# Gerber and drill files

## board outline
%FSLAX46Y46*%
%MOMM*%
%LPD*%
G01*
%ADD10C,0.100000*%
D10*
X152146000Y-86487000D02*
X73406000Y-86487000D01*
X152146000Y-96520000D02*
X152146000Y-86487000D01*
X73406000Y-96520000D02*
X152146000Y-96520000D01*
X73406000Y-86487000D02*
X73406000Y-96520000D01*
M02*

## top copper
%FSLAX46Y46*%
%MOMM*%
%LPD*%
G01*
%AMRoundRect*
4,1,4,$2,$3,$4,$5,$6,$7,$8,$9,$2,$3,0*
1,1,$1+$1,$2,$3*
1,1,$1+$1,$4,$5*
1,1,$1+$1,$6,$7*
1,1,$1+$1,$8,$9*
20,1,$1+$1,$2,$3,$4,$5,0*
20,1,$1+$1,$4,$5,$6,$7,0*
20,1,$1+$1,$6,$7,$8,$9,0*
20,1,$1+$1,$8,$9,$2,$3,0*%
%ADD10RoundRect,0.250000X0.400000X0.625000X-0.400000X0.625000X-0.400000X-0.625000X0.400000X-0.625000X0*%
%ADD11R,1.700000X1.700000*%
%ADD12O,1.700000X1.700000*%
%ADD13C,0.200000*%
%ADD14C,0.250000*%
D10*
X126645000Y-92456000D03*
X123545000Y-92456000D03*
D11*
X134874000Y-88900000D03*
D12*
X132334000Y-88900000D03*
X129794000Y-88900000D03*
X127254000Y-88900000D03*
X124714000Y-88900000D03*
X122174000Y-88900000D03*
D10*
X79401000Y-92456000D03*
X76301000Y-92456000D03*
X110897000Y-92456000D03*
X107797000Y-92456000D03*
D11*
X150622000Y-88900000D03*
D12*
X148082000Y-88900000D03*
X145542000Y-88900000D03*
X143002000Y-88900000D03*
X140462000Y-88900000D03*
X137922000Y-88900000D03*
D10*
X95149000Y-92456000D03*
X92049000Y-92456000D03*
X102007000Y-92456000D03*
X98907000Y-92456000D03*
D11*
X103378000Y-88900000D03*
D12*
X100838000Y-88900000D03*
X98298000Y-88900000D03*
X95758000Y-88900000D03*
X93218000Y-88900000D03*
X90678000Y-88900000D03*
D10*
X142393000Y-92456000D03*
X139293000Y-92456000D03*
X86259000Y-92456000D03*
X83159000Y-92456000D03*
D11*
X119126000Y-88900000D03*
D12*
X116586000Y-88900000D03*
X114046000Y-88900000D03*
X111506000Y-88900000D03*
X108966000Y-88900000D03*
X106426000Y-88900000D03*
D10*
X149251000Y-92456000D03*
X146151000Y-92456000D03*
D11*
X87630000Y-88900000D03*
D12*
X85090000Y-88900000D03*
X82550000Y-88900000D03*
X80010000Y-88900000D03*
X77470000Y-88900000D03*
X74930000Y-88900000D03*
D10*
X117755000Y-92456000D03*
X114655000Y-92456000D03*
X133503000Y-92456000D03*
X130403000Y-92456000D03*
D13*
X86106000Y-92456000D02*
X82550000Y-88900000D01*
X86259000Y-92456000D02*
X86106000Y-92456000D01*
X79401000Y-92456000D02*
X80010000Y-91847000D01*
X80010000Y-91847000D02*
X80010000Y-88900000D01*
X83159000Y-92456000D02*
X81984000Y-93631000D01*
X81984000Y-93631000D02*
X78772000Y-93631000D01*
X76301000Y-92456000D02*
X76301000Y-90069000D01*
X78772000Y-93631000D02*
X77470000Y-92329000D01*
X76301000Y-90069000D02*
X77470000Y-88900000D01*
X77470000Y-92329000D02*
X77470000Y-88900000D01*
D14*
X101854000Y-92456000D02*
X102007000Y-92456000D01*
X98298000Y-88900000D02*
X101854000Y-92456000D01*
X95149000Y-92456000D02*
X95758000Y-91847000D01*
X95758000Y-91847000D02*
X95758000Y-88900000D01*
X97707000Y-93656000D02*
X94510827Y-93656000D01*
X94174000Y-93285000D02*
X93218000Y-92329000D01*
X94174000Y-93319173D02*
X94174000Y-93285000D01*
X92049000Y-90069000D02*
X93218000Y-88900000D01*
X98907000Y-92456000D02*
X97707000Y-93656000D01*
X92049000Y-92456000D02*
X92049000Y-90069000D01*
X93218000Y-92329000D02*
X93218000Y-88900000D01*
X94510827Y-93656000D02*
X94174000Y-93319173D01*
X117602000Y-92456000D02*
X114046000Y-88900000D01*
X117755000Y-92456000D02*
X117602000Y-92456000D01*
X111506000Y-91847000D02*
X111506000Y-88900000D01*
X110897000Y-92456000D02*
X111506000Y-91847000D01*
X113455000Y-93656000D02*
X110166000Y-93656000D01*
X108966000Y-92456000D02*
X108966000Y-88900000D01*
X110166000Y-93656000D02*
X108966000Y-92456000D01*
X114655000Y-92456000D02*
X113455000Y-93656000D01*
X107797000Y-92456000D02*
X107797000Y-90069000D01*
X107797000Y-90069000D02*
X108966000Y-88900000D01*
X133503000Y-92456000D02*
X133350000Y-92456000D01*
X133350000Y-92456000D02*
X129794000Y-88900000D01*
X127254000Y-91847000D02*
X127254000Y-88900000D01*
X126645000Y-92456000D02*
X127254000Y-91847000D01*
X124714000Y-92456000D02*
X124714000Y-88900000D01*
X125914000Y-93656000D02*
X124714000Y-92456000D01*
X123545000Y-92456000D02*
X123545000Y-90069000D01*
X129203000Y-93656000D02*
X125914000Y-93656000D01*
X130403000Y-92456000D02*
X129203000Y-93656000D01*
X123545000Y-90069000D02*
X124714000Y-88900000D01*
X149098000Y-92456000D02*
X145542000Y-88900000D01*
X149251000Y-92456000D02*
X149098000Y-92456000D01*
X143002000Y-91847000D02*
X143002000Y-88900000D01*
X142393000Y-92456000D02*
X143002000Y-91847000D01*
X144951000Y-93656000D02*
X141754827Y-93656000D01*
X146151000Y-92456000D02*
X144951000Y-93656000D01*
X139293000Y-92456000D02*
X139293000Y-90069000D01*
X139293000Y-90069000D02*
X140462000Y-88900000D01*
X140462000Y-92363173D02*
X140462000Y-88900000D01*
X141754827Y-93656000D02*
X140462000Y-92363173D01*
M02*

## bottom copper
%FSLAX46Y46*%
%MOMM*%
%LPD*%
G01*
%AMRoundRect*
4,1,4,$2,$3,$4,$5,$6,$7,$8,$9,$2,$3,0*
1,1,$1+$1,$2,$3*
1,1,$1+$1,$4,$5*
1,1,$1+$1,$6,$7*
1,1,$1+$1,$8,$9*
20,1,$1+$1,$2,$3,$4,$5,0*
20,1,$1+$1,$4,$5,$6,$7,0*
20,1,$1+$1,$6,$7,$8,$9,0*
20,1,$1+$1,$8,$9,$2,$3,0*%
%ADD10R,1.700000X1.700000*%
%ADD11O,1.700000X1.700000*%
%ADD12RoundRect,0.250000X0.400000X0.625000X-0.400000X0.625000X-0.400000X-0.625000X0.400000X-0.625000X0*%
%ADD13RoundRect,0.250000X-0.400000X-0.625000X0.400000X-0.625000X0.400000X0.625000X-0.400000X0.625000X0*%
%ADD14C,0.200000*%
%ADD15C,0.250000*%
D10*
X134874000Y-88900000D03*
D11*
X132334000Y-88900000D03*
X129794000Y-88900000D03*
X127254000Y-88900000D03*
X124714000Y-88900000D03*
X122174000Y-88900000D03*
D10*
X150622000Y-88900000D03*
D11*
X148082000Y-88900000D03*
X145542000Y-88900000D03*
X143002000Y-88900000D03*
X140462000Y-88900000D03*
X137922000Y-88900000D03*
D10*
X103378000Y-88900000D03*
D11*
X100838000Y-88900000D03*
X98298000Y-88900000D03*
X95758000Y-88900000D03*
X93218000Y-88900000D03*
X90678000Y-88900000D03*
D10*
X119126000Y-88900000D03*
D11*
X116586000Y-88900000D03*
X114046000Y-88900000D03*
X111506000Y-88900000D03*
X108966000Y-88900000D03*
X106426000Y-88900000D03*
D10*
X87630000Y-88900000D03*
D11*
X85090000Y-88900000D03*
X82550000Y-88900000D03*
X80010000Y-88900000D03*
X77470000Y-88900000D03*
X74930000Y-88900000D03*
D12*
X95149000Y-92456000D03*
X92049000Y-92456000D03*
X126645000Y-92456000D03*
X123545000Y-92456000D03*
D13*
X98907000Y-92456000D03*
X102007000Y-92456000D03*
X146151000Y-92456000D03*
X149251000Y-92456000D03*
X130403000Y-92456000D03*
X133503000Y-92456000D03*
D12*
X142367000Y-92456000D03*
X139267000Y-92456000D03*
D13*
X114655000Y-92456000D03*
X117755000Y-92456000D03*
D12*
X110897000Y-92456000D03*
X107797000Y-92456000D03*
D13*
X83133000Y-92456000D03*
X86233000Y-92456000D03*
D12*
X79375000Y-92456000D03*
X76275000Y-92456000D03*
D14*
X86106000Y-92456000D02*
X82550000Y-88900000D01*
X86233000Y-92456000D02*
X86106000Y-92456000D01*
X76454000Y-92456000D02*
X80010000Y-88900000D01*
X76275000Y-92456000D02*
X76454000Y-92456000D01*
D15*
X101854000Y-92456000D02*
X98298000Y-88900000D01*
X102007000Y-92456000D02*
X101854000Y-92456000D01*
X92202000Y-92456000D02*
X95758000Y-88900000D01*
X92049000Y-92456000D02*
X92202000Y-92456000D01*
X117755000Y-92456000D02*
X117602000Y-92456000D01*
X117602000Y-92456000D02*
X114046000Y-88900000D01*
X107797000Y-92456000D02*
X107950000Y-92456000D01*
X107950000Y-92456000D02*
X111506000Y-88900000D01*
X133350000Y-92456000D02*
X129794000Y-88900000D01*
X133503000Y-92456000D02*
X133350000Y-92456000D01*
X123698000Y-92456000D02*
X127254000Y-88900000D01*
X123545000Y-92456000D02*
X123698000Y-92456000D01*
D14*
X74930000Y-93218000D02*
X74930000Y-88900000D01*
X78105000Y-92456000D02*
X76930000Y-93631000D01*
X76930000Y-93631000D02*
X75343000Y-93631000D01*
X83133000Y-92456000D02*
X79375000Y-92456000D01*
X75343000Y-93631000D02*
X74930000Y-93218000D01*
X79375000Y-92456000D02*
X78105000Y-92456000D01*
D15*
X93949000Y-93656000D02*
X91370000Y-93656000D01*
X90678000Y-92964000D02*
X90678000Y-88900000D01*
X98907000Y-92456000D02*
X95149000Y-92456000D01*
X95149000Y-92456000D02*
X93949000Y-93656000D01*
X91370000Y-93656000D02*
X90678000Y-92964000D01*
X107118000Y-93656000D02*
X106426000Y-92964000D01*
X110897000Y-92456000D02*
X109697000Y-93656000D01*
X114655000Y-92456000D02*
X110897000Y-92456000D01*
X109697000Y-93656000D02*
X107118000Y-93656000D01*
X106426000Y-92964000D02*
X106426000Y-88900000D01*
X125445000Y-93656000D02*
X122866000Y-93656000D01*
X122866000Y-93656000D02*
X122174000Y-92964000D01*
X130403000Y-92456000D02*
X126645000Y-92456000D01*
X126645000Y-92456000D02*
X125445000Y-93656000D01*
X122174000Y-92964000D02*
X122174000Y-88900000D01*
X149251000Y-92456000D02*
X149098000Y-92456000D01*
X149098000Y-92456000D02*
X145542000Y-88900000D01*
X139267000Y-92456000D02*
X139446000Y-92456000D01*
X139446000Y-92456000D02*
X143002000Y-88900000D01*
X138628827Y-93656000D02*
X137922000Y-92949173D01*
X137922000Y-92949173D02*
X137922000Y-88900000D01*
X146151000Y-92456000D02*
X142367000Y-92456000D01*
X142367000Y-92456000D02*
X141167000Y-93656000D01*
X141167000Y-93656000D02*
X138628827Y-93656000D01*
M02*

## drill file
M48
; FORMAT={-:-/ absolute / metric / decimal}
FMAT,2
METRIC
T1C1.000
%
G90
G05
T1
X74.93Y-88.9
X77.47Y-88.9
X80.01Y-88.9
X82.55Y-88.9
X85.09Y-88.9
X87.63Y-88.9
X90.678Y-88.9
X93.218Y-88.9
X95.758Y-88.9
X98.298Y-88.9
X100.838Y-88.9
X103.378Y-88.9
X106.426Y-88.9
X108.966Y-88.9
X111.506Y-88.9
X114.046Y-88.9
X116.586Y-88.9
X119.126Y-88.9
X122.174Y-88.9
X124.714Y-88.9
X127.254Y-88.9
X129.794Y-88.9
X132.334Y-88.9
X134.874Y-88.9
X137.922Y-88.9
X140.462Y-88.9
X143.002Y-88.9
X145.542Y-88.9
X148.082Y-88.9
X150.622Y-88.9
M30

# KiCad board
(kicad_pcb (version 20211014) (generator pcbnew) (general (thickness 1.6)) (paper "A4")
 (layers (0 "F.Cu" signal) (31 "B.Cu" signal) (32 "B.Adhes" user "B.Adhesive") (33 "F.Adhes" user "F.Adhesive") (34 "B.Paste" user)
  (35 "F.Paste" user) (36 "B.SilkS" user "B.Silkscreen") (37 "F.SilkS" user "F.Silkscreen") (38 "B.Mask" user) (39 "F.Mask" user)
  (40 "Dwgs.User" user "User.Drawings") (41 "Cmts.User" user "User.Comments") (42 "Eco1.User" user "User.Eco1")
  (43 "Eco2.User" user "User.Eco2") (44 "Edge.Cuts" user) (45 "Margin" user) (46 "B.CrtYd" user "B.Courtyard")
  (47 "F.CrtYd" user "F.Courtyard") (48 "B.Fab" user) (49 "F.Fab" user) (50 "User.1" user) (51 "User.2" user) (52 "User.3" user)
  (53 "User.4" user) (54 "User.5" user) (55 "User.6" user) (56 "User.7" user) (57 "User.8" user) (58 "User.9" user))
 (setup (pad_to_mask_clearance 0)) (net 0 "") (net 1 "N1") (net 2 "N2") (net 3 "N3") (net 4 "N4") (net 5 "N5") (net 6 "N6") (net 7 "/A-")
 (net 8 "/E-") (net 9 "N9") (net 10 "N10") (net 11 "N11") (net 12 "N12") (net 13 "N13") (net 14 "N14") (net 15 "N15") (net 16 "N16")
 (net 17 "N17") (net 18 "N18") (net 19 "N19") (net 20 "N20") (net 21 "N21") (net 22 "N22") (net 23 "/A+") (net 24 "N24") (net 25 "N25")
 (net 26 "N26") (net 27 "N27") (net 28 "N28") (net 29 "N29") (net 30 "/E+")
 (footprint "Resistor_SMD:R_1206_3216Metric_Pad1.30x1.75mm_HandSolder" (layer "F.Cu") (at 125.095 92.456 180)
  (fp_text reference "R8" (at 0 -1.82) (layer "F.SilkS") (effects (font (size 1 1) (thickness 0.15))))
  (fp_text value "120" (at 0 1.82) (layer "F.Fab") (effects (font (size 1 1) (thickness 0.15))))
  (pad "1" smd roundrect (at -1.55 0 180) (size 1.3 1.75) (layers "F.Cu" "F.Paste" "F.Mask") (roundrect_rratio 0.1923076923) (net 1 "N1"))
  (pad "2" smd roundrect (at 1.55 0 180) (size 1.3 1.75) (layers "F.Cu" "F.Paste" "F.Mask") (roundrect_rratio 0.1923076923) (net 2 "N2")))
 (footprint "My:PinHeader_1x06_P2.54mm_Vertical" (layer "F.Cu") (at 134.874 88.9 -90)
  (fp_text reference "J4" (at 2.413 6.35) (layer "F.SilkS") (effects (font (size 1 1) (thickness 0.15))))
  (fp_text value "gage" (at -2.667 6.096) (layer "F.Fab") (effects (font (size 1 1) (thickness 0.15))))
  (pad "1" thru_hole rect (at 0 0 270) (size 1.7 1.7) (drill 1) (layers *.Cu *.Mask) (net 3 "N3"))
  (pad "2" thru_hole oval (at 0 2.54 270) (size 1.7 1.7) (drill 1) (layers *.Cu *.Mask) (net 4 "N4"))
  (pad "3" thru_hole oval (at 0 5.08 270) (size 1.7 1.7) (drill 1) (layers *.Cu *.Mask) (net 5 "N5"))
  (pad "4" thru_hole oval (at 0 7.62 270) (size 1.7 1.7) (drill 1) (layers *.Cu *.Mask) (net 1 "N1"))
  (pad "5" thru_hole oval (at 0 10.16 270) (size 1.7 1.7) (drill 1) (layers *.Cu *.Mask) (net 2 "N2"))
  (pad "6" thru_hole oval (at 0 12.7 270) (size 1.7 1.7) (drill 1) (layers *.Cu *.Mask) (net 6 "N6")))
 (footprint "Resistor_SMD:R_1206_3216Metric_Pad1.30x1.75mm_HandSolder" (layer "F.Cu") (at 77.851 92.456 180)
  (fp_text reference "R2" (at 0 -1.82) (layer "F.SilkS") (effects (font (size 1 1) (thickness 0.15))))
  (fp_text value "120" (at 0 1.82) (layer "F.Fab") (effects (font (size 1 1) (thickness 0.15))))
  (pad "1" smd roundrect (at -1.55 0 180) (size 1.3 1.75) (layers "F.Cu" "F.Paste" "F.Mask") (roundrect_rratio 0.1923076923) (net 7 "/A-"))
  (pad "2" smd roundrect (at 1.55 0 180) (size 1.3 1.75) (layers "F.Cu" "F.Paste" "F.Mask") (roundrect_rratio 0.1923076923) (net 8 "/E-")))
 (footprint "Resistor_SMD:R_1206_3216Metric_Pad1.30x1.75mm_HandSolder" (layer "F.Cu") (at 109.347 92.456 180)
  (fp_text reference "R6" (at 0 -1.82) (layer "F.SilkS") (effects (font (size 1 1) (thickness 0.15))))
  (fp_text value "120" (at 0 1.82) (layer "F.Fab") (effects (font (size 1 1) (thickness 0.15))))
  (pad "1" smd roundrect (at -1.55 0 180) (size 1.3 1.75) (layers "F.Cu" "F.Paste" "F.Mask") (roundrect_rratio 0.1923076923) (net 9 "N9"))
  (pad "2" smd roundrect (at 1.55 0 180) (size 1.3 1.75) (layers "F.Cu" "F.Paste" "F.Mask") (roundrect_rratio 0.1923076923) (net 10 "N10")))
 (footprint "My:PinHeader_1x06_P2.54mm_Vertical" (layer "F.Cu") (at 150.622 88.9 -90)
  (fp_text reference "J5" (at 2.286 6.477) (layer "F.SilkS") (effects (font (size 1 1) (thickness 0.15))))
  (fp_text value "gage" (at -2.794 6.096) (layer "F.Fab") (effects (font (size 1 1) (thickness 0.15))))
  (pad "1" thru_hole rect (at 0 0 270) (size 1.7 1.7) (drill 1) (layers *.Cu *.Mask) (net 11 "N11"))
  (pad "2" thru_hole oval (at 0 2.54 270) (size 1.7 1.7) (drill 1) (layers *.Cu *.Mask) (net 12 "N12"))
  (pad "3" thru_hole oval (at 0 5.08 270) (size 1.7 1.7) (drill 1) (layers *.Cu *.Mask) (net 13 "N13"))
  (pad "4" thru_hole oval (at 0 7.62 270) (size 1.7 1.7) (drill 1) (layers *.Cu *.Mask) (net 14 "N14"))
  (pad "5" thru_hole oval (at 0 10.16 270) (size 1.7 1.7) (drill 1) (layers *.Cu *.Mask) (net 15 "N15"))
  (pad "6" thru_hole oval (at 0 12.7 270) (size 1.7 1.7) (drill 1) (layers *.Cu *.Mask) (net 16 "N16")))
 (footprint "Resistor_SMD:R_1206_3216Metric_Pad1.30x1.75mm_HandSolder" (layer "F.Cu") (at 93.599 92.456 180)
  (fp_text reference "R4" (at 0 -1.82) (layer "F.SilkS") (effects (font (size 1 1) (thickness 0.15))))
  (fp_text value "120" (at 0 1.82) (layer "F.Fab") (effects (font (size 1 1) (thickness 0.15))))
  (pad "1" smd roundrect (at -1.55 0 180) (size 1.3 1.75) (layers "F.Cu" "F.Paste" "F.Mask") (roundrect_rratio 0.1923076923) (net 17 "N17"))
  (pad "2" smd roundrect (at 1.55 0 180) (size 1.3 1.75) (layers "F.Cu" "F.Paste" "F.Mask") (roundrect_rratio 0.1923076923) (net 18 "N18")))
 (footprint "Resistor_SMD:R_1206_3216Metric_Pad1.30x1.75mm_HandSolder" (layer "F.Cu") (at 100.457 92.456 180)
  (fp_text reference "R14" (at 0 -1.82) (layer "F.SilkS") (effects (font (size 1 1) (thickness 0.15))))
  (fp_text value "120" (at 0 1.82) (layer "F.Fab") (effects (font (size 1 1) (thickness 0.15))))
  (pad "1" smd roundrect (at -1.55 0 180) (size 1.3 1.75) (layers "F.Cu" "F.Paste" "F.Mask") (roundrect_rratio 0.1923076923) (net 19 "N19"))
  (pad "2" smd roundrect (at 1.55 0 180) (size 1.3 1.75) (layers "F.Cu" "F.Paste" "F.Mask") (roundrect_rratio 0.1923076923) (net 18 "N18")))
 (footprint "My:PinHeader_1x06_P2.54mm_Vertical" (layer "F.Cu") (at 103.378 88.9 -90)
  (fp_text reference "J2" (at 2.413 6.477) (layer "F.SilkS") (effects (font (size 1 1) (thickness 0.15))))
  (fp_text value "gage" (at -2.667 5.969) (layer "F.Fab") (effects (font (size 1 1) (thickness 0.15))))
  (pad "1" thru_hole rect (at 0 0 270) (size 1.7 1.7) (drill 1) (layers *.Cu *.Mask) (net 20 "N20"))
  (pad "2" thru_hole oval (at 0 2.54 270) (size 1.7 1.7) (drill 1) (layers *.Cu *.Mask) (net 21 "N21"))
  (pad "3" thru_hole oval (at 0 5.08 270) (size 1.7 1.7) (drill 1) (layers *.Cu *.Mask) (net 19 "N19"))
  (pad "4" thru_hole oval (at 0 7.62 270) (size 1.7 1.7) (drill 1) (layers *.Cu *.Mask) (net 17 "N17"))
  (pad "5" thru_hole oval (at 0 10.16 270) (size 1.7 1.7) (drill 1) (layers *.Cu *.Mask) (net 18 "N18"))
  (pad "6" thru_hole oval (at 0 12.7 270) (size 1.7 1.7) (drill 1) (layers *.Cu *.Mask) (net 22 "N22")))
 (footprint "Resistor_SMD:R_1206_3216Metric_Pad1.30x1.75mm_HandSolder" (layer "F.Cu") (at 140.843 92.456 180)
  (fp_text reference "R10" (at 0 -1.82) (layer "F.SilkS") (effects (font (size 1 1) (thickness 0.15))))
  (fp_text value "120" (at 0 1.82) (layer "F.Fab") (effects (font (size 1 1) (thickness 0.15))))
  (pad "1" smd roundrect (at -1.55 0 180) (size 1.3 1.75) (layers "F.Cu" "F.Paste" "F.Mask") (roundrect_rratio 0.1923076923) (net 14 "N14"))
  (pad "2" smd roundrect (at 1.55 0 180) (size 1.3 1.75) (layers "F.Cu" "F.Paste" "F.Mask") (roundrect_rratio 0.1923076923) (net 15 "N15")))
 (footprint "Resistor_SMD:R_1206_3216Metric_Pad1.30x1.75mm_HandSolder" (layer "F.Cu") (at 84.709 92.456 180)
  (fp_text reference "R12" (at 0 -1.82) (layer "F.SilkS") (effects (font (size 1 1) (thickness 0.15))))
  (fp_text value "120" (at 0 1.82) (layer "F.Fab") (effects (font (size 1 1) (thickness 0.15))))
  (pad "1" smd roundrect (at -1.55 0 180) (size 1.3 1.75) (layers "F.Cu" "F.Paste" "F.Mask") (roundrect_rratio 0.1923076923) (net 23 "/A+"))
  (pad "2" smd roundrect (at 1.55 0 180) (size 1.3 1.75) (layers "F.Cu" "F.Paste" "F.Mask") (roundrect_rratio 0.1923076923) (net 8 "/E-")))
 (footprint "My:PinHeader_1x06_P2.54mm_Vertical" (layer "F.Cu") (at 119.126 88.9 -90)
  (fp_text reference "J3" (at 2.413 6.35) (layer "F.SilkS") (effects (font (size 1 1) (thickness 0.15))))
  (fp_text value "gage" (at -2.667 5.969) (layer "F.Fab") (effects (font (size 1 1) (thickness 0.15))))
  (pad "1" thru_hole rect (at 0 0 270) (size 1.7 1.7) (drill 1) (layers *.Cu *.Mask) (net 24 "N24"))
  (pad "2" thru_hole oval (at 0 2.54 270) (size 1.7 1.7) (drill 1) (layers *.Cu *.Mask) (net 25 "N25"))
  (pad "3" thru_hole oval (at 0 5.08 270) (size 1.7 1.7) (drill 1) (layers *.Cu *.Mask) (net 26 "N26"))
  (pad "4" thru_hole oval (at 0 7.62 270) (size 1.7 1.7) (drill 1) (layers *.Cu *.Mask) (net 9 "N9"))
  (pad "5" thru_hole oval (at 0 10.16 270) (size 1.7 1.7) (drill 1) (layers *.Cu *.Mask) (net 10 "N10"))
  (pad "6" thru_hole oval (at 0 12.7 270) (size 1.7 1.7) (drill 1) (layers *.Cu *.Mask) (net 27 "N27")))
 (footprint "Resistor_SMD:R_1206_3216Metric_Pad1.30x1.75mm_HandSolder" (layer "F.Cu") (at 147.701 92.456 180)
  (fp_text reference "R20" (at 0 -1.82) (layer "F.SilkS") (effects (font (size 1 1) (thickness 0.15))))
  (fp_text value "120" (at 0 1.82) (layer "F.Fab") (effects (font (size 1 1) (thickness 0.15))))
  (pad "1" smd roundrect (at -1.55 0 180) (size 1.3 1.75) (layers "F.Cu" "F.Paste" "F.Mask") (roundrect_rratio 0.1923076923) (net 13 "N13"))
  (pad "2" smd roundrect (at 1.55 0 180) (size 1.3 1.75) (layers "F.Cu" "F.Paste" "F.Mask") (roundrect_rratio 0.1923076923) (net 15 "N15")))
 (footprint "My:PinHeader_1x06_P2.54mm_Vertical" (layer "F.Cu") (at 87.63 88.9 -90)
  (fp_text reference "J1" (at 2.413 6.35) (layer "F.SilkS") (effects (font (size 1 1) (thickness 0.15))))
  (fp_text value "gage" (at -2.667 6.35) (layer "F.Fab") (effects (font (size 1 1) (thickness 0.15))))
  (pad "1" thru_hole rect (at 0 0 270) (size 1.7 1.7) (drill 1) (layers *.Cu *.Mask) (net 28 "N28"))
  (pad "2" thru_hole oval (at 0 2.54 270) (size 1.7 1.7) (drill 1) (layers *.Cu *.Mask) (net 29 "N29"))
  (pad "3" thru_hole oval (at 0 5.08 270) (size 1.7 1.7) (drill 1) (layers *.Cu *.Mask) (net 23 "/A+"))
  (pad "4" thru_hole oval (at 0 7.62 270) (size 1.7 1.7) (drill 1) (layers *.Cu *.Mask) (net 7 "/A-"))
  (pad "5" thru_hole oval (at 0 10.16 270) (size 1.7 1.7) (drill 1) (layers *.Cu *.Mask) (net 8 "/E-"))
  (pad "6" thru_hole oval (at 0 12.7 270) (size 1.7 1.7) (drill 1) (layers *.Cu *.Mask) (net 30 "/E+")))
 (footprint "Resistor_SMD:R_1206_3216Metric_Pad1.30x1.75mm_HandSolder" (layer "F.Cu") (at 116.205 92.456 180)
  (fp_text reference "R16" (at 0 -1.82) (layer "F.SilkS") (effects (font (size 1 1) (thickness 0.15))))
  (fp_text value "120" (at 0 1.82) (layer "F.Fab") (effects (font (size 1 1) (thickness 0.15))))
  (pad "1" smd roundrect (at -1.55 0 180) (size 1.3 1.75) (layers "F.Cu" "F.Paste" "F.Mask") (roundrect_rratio 0.1923076923) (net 26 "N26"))
  (pad "2" smd roundrect (at 1.55 0 180) (size 1.3 1.75) (layers "F.Cu" "F.Paste" "F.Mask") (roundrect_rratio 0.1923076923) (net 10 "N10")))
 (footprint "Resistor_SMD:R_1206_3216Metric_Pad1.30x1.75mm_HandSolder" (layer "F.Cu") (at 131.953 92.456 180)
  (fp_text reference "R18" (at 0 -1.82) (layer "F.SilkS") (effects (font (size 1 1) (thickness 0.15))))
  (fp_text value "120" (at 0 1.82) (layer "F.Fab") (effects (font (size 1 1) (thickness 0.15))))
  (pad "1" smd roundrect (at -1.55 0 180) (size 1.3 1.75) (layers "F.Cu" "F.Paste" "F.Mask") (roundrect_rratio 0.1923076923) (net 5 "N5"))
  (pad "2" smd roundrect (at 1.55 0 180) (size 1.3 1.75) (layers "F.Cu" "F.Paste" "F.Mask") (roundrect_rratio 0.1923076923) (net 2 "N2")))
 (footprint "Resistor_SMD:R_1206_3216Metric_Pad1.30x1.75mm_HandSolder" (layer "B.Cu") (at 93.599 92.456 180)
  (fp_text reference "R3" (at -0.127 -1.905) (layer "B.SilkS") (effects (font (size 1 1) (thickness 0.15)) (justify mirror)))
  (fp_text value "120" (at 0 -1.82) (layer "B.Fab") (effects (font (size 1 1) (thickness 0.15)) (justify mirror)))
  (pad "1" smd roundrect (at -1.55 0 180) (size 1.3 1.75) (layers "B.Cu" "B.Paste" "B.Mask") (roundrect_rratio 0.1923076923) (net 22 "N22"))
  (pad "2" smd roundrect (at 1.55 0 180) (size 1.3 1.75) (layers "B.Cu" "B.Paste" "B.Mask") (roundrect_rratio 0.1923076923) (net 17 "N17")))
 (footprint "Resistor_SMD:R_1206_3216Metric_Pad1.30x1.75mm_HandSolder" (layer "B.Cu") (at 125.095 92.456 180)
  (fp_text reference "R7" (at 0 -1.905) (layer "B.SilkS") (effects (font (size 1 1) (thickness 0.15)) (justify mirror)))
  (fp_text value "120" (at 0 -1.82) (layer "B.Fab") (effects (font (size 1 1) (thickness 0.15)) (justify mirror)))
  (pad "1" smd roundrect (at -1.55 0 180) (size 1.3 1.75) (layers "B.Cu" "B.Paste" "B.Mask") (roundrect_rratio 0.1923076923) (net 6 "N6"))
  (pad "2" smd roundrect (at 1.55 0 180) (size 1.3 1.75) (layers "B.Cu" "B.Paste" "B.Mask") (roundrect_rratio 0.1923076923) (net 1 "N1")))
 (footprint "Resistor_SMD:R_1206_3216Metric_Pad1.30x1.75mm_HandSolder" (layer "B.Cu") (at 100.457 92.456)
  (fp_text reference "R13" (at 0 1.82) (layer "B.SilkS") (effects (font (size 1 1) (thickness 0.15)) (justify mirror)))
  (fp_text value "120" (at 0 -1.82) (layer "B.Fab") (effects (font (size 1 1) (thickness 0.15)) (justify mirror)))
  (pad "1" smd roundrect (at -1.55 0) (size 1.3 1.75) (layers "B.Cu" "B.Paste" "B.Mask") (roundrect_rratio 0.1923076923) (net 22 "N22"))
  (pad "2" smd roundrect (at 1.55 0) (size 1.3 1.75) (layers "B.Cu" "B.Paste" "B.Mask") (roundrect_rratio 0.1923076923) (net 19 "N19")))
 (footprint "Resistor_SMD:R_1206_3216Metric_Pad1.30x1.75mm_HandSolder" (layer "B.Cu") (at 147.701 92.456)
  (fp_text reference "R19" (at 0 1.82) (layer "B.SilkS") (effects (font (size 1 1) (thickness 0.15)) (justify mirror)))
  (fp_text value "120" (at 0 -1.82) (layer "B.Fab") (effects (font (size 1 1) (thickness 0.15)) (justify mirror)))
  (pad "1" smd roundrect (at -1.55 0) (size 1.3 1.75) (layers "B.Cu" "B.Paste" "B.Mask") (roundrect_rratio 0.1923076923) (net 16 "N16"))
  (pad "2" smd roundrect (at 1.55 0) (size 1.3 1.75) (layers "B.Cu" "B.Paste" "B.Mask") (roundrect_rratio 0.1923076923) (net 13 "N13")))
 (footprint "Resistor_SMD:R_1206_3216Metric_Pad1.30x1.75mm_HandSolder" (layer "B.Cu") (at 131.953 92.456)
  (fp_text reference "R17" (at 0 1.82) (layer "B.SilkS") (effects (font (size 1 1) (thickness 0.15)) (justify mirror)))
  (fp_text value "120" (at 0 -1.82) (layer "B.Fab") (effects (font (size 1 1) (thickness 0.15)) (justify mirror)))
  (pad "1" smd roundrect (at -1.55 0) (size 1.3 1.75) (layers "B.Cu" "B.Paste" "B.Mask") (roundrect_rratio 0.1923076923) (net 6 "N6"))
  (pad "2" smd roundrect (at 1.55 0) (size 1.3 1.75) (layers "B.Cu" "B.Paste" "B.Mask") (roundrect_rratio 0.1923076923) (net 5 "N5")))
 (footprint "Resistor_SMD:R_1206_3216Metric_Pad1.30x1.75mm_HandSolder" (layer "B.Cu") (at 140.817 92.456 180)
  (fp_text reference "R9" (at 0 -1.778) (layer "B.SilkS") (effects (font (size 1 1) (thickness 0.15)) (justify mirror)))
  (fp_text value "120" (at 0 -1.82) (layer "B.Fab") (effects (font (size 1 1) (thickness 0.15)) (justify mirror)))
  (pad "1" smd roundrect (at -1.55 0 180) (size 1.3 1.75) (layers "B.Cu" "B.Paste" "B.Mask") (roundrect_rratio 0.1923076923) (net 16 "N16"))
  (pad "2" smd roundrect (at 1.55 0 180) (size 1.3 1.75) (layers "B.Cu" "B.Paste" "B.Mask") (roundrect_rratio 0.1923076923) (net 14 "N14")))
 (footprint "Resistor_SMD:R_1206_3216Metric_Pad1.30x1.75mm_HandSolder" (layer "B.Cu") (at 116.205 92.456)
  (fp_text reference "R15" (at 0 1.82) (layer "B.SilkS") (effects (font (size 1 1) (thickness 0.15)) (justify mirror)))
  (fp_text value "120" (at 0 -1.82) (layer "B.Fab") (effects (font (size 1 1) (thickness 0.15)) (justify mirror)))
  (pad "1" smd roundrect (at -1.55 0) (size 1.3 1.75) (layers "B.Cu" "B.Paste" "B.Mask") (roundrect_rratio 0.1923076923) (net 27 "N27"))
  (pad "2" smd roundrect (at 1.55 0) (size 1.3 1.75) (layers "B.Cu" "B.Paste" "B.Mask") (roundrect_rratio 0.1923076923) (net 26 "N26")))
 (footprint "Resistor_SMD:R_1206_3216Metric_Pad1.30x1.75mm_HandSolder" (layer "B.Cu") (at 109.347 92.456 180)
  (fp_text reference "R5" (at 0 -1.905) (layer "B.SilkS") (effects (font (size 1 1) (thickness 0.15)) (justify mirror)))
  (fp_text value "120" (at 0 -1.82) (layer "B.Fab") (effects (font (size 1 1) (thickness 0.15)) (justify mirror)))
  (pad "1" smd roundrect (at -1.55 0 180) (size 1.3 1.75) (layers "B.Cu" "B.Paste" "B.Mask") (roundrect_rratio 0.1923076923) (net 27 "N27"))
  (pad "2" smd roundrect (at 1.55 0 180) (size 1.3 1.75) (layers "B.Cu" "B.Paste" "B.Mask") (roundrect_rratio 0.1923076923) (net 9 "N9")))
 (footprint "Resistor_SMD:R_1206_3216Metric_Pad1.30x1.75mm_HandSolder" (layer "B.Cu") (at 84.683 92.456)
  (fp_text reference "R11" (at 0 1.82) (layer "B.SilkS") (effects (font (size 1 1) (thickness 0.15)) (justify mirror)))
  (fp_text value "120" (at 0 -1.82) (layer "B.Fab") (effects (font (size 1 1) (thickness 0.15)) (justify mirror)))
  (pad "1" smd roundrect (at -1.55 0) (size 1.3 1.75) (layers "B.Cu" "B.Paste" "B.Mask") (roundrect_rratio 0.1923076923) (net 30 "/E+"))
  (pad "2" smd roundrect (at 1.55 0) (size 1.3 1.75) (layers "B.Cu" "B.Paste" "B.Mask") (roundrect_rratio 0.1923076923) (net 23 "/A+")))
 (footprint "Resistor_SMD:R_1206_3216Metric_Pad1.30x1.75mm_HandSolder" (layer "B.Cu") (at 77.825 92.456 180)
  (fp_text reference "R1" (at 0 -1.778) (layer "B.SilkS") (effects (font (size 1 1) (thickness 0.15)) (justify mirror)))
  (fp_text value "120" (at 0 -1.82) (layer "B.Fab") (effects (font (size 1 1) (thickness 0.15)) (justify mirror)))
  (pad "1" smd roundrect (at -1.55 0 180) (size 1.3 1.75) (layers "B.Cu" "B.Paste" "B.Mask") (roundrect_rratio 0.1923076923) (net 30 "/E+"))
  (pad "2" smd roundrect (at 1.55 0 180) (size 1.3 1.75) (layers "B.Cu" "B.Paste" "B.Mask") (roundrect_rratio 0.1923076923) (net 7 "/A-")))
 (gr_line (start 152.146 86.487) (end 73.406 86.487) (layer "Edge.Cuts") (width 0.1))
 (gr_line (start 152.146 96.52) (end 152.146 86.487) (layer "Edge.Cuts") (width 0.1))
 (gr_line (start 73.406 96.52) (end 152.146 96.52) (layer "Edge.Cuts") (width 0.1))
 (gr_line (start 73.406 86.487) (end 73.406 96.52) (layer "Edge.Cuts") (width 0.1))
 (segment (start 86.106 92.456) (end 82.55 88.9) (width 0.2) (layer "F.Cu") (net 23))
 (segment (start 86.259 92.456) (end 86.106 92.456) (width 0.2) (layer "F.Cu") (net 23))
 (segment (start 86.106 92.456) (end 82.55 88.9) (width 0.2) (layer "B.Cu") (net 23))
 (segment (start 86.233 92.456) (end 86.106 92.456) (width 0.2) (layer "B.Cu") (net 23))
 (segment (start 79.401 92.456) (end 80.01 91.847) (width 0.2) (layer "F.Cu") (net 7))
 (segment (start 80.01 91.847) (end 80.01 88.9) (width 0.2) (layer "F.Cu") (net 7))
 (segment (start 76.454 92.456) (end 80.01 88.9) (width 0.2) (layer "B.Cu") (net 7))
 (segment (start 76.275 92.456) (end 76.454 92.456) (width 0.2) (layer "B.Cu") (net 7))
 (segment (start 83.159 92.456) (end 81.984 93.631) (width 0.2) (layer "F.Cu") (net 8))
 (segment (start 81.984 93.631) (end 78.772 93.631) (width 0.2) (layer "F.Cu") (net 8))
 (segment (start 76.301 92.456) (end 76.301 90.069) (width 0.2) (layer "F.Cu") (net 8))
 (segment (start 78.772 93.631) (end 77.47 92.329) (width 0.2) (layer "F.Cu") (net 8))
 (segment (start 76.301 90.069) (end 77.47 88.9) (width 0.2) (layer "F.Cu") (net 8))
 (segment (start 77.47 92.329) (end 77.47 88.9) (width 0.2) (layer "F.Cu") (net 8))
 (segment (start 101.854 92.456) (end 102.007 92.456) (width 0.25) (layer "F.Cu") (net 19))
 (segment (start 98.298 88.9) (end 101.854 92.456) (width 0.25) (layer "F.Cu") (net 19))
 (segment (start 101.854 92.456) (end 98.298 88.9) (width 0.25) (layer "B.Cu") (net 19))
 (segment (start 102.007 92.456) (end 101.854 92.456) (width 0.25) (layer "B.Cu") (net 19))
 (segment (start 95.149 92.456) (end 95.758 91.847) (width 0.25) (layer "F.Cu") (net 17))
 (segment (start 95.758 91.847) (end 95.758 88.9) (width 0.25) (layer "F.Cu") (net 17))
 (segment (start 92.202 92.456) (end 95.758 88.9) (width 0.25) (layer "B.Cu") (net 17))
 (segment (start 92.049 92.456) (end 92.202 92.456) (width 0.25) (layer "B.Cu") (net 17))
 (segment (start 97.707 93.656) (end 94.510827 93.656) (width 0.25) (layer "F.Cu") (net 18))
 (segment (start 94.174 93.285) (end 93.218 92.329) (width 0.25) (layer "F.Cu") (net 18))
 (segment (start 94.174 93.319173) (end 94.174 93.285) (width 0.25) (layer "F.Cu") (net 18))
 (segment (start 92.049 90.069) (end 93.218 88.9) (width 0.25) (layer "F.Cu") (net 18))
 (segment (start 98.907 92.456) (end 97.707 93.656) (width 0.25) (layer "F.Cu") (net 18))
 (segment (start 92.049 92.456) (end 92.049 90.069) (width 0.25) (layer "F.Cu") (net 18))
 (segment (start 93.218 92.329) (end 93.218 88.9) (width 0.25) (layer "F.Cu") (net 18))
 (segment (start 94.510827 93.656) (end 94.174 93.319173) (width 0.25) (layer "F.Cu") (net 18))
 (segment (start 117.602 92.456) (end 114.046 88.9) (width 0.25) (layer "F.Cu") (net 26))
 (segment (start 117.755 92.456) (end 117.602 92.456) (width 0.25) (layer "F.Cu") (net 26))
 (segment (start 117.755 92.456) (end 117.602 92.456) (width 0.25) (layer "B.Cu") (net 26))
 (segment (start 117.602 92.456) (end 114.046 88.9) (width 0.25) (layer "B.Cu") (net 26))
 (segment (start 111.506 91.847) (end 111.506 88.9) (width 0.25) (layer "F.Cu") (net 9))
 (segment (start 110.897 92.456) (end 111.506 91.847) (width 0.25) (layer "F.Cu") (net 9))
 (segment (start 107.797 92.456) (end 107.95 92.456) (width 0.25) (layer "B.Cu") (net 9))
 (segment (start 107.95 92.456) (end 111.506 88.9) (width 0.25) (layer "B.Cu") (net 9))
 (segment (start 113.455 93.656) (end 110.166 93.656) (width 0.25) (layer "F.Cu") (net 10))
 (segment (start 108.966 92.456) (end 108.966 88.9) (width 0.25) (layer "F.Cu") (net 10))
 (segment (start 110.166 93.656) (end 108.966 92.456) (width 0.25) (layer "F.Cu") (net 10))
 (segment (start 114.655 92.456) (end 113.455 93.656) (width 0.25) (layer "F.Cu") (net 10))
 (segment (start 107.797 92.456) (end 107.797 90.069) (width 0.25) (layer "F.Cu") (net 10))
 (segment (start 107.797 90.069) (end 108.966 88.9) (width 0.25) (layer "F.Cu") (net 10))
 (segment (start 133.503 92.456) (end 133.35 92.456) (width 0.25) (layer "F.Cu") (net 5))
 (segment (start 133.35 92.456) (end 129.794 88.9) (width 0.25) (layer "F.Cu") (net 5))
 (segment (start 133.35 92.456) (end 129.794 88.9) (width 0.25) (layer "B.Cu") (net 5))
 (segment (start 133.503 92.456) (end 133.35 92.456) (width 0.25) (layer "B.Cu") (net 5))
 (segment (start 127.254 91.847) (end 127.254 88.9) (width 0.25) (layer "F.Cu") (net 1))
 (segment (start 126.645 92.456) (end 127.254 91.847) (width 0.25) (layer "F.Cu") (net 1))
 (segment (start 123.698 92.456) (end 127.254 88.9) (width 0.25) (layer "B.Cu") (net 1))
 (segment (start 123.545 92.456) (end 123.698 92.456) (width 0.25) (layer "B.Cu") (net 1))
 (segment (start 124.714 92.456) (end 124.714 88.9) (width 0.25) (layer "F.Cu") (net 2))
 (segment (start 125.914 93.656) (end 124.714 92.456) (width 0.25) (layer "F.Cu") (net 2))
 (segment (start 123.545 92.456) (end 123.545 90.069) (width 0.25) (layer "F.Cu") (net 2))
 (segment (start 129.203 93.656) (end 125.914 93.656) (width 0.25) (layer "F.Cu") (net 2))
 (segment (start 130.403 92.456) (end 129.203 93.656) (width 0.25) (layer "F.Cu") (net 2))
 (segment (start 123.545 90.069) (end 124.714 88.9) (width 0.25) (layer "F.Cu") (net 2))
 (segment (start 74.93 93.218) (end 74.93 88.9) (width 0.2) (layer "B.Cu") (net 30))
 (segment (start 78.105 92.456) (end 76.93 93.631) (width 0.2) (layer "B.Cu") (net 30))
 (segment (start 76.93 93.631) (end 75.343 93.631) (width 0.2) (layer "B.Cu") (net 30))
 (segment (start 83.133 92.456) (end 79.375 92.456) (width 0.2) (layer "B.Cu") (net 30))
 (segment (start 75.343 93.631) (end 74.93 93.218) (width 0.2) (layer "B.Cu") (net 30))
 (segment (start 79.375 92.456) (end 78.105 92.456) (width 0.2) (layer "B.Cu") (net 30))
 (segment (start 93.949 93.656) (end 91.37 93.656) (width 0.25) (layer "B.Cu") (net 22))
 (segment (start 90.678 92.964) (end 90.678 88.9) (width 0.25) (layer "B.Cu") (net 22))
 (segment (start 98.907 92.456) (end 95.149 92.456) (width 0.25) (layer "B.Cu") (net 22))
 (segment (start 95.149 92.456) (end 93.949 93.656) (width 0.25) (layer "B.Cu") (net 22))
 (segment (start 91.37 93.656) (end 90.678 92.964) (width 0.25) (layer "B.Cu") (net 22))
 (segment (start 107.118 93.656) (end 106.426 92.964) (width 0.25) (layer "B.Cu") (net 27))
 (segment (start 110.897 92.456) (end 109.697 93.656) (width 0.25) (layer "B.Cu") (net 27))
 (segment (start 114.655 92.456) (end 110.897 92.456) (width 0.25) (layer "B.Cu") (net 27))
 (segment (start 109.697 93.656) (end 107.118 93.656) (width 0.25) (layer "B.Cu") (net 27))
 (segment (start 106.426 92.964) (end 106.426 88.9) (width 0.25) (layer "B.Cu") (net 27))
 (segment (start 125.445 93.656) (end 122.866 93.656) (width 0.25) (layer "B.Cu") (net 6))
 (segment (start 122.866 93.656) (end 122.174 92.964) (width 0.25) (layer "B.Cu") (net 6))
 (segment (start 130.403 92.456) (end 126.645 92.456) (width 0.25) (layer "B.Cu") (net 6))
 (segment (start 126.645 92.456) (end 125.445 93.656) (width 0.25) (layer "B.Cu") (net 6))
 (segment (start 122.174 92.964) (end 122.174 88.9) (width 0.25) (layer "B.Cu") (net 6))
 (segment (start 149.098 92.456) (end 145.542 88.9) (width 0.25) (layer "F.Cu") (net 13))
 (segment (start 149.251 92.456) (end 149.098 92.456) (width 0.25) (layer "F.Cu") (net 13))
 (segment (start 149.251 92.456) (end 149.098 92.456) (width 0.25) (layer "B.Cu") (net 13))
 (segment (start 149.098 92.456) (end 145.542 88.9) (width 0.25) (layer "B.Cu") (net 13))
 (segment (start 143.002 91.847) (end 143.002 88.9) (width 0.25) (layer "F.Cu") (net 14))
 (segment (start 142.393 92.456) (end 143.002 91.847) (width 0.25) (layer "F.Cu") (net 14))
 (segment (start 139.267 92.456) (end 139.446 92.456) (width 0.25) (layer "B.Cu") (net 14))
 (segment (start 139.446 92.456) (end 143.002 88.9) (width 0.25) (layer "B.Cu") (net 14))
 (segment (start 144.951 93.656) (end 141.754827 93.656) (width 0.25) (layer "F.Cu") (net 15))
 (segment (start 146.151 92.456) (end 144.951 93.656) (width 0.25) (layer "F.Cu") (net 15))
 (segment (start 139.293 92.456) (end 139.293 90.069) (width 0.25) (layer "F.Cu") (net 15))
 (segment (start 139.293 90.069) (end 140.462 88.9) (width 0.25) (layer "F.Cu") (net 15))
 (segment (start 140.462 92.363173) (end 140.462 88.9) (width 0.25) (layer "F.Cu") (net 15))
 (segment (start 141.754827 93.656) (end 140.462 92.363173) (width 0.25) (layer "F.Cu") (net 15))
 (segment (start 138.628827 93.656) (end 137.922 92.949173) (width 0.25) (layer "B.Cu") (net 16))
 (segment (start 137.922 92.949173) (end 137.922 88.9) (width 0.25) (layer "B.Cu") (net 16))
 (segment (start 146.151 92.456) (end 142.367 92.456) (width 0.25) (layer "B.Cu") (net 16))
 (segment (start 142.367 92.456) (end 141.167 93.656) (width 0.25) (layer "B.Cu") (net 16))
 (segment (start 141.167 93.656) (end 138.628827 93.656) (width 0.25) (layer "B.Cu") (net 16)))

